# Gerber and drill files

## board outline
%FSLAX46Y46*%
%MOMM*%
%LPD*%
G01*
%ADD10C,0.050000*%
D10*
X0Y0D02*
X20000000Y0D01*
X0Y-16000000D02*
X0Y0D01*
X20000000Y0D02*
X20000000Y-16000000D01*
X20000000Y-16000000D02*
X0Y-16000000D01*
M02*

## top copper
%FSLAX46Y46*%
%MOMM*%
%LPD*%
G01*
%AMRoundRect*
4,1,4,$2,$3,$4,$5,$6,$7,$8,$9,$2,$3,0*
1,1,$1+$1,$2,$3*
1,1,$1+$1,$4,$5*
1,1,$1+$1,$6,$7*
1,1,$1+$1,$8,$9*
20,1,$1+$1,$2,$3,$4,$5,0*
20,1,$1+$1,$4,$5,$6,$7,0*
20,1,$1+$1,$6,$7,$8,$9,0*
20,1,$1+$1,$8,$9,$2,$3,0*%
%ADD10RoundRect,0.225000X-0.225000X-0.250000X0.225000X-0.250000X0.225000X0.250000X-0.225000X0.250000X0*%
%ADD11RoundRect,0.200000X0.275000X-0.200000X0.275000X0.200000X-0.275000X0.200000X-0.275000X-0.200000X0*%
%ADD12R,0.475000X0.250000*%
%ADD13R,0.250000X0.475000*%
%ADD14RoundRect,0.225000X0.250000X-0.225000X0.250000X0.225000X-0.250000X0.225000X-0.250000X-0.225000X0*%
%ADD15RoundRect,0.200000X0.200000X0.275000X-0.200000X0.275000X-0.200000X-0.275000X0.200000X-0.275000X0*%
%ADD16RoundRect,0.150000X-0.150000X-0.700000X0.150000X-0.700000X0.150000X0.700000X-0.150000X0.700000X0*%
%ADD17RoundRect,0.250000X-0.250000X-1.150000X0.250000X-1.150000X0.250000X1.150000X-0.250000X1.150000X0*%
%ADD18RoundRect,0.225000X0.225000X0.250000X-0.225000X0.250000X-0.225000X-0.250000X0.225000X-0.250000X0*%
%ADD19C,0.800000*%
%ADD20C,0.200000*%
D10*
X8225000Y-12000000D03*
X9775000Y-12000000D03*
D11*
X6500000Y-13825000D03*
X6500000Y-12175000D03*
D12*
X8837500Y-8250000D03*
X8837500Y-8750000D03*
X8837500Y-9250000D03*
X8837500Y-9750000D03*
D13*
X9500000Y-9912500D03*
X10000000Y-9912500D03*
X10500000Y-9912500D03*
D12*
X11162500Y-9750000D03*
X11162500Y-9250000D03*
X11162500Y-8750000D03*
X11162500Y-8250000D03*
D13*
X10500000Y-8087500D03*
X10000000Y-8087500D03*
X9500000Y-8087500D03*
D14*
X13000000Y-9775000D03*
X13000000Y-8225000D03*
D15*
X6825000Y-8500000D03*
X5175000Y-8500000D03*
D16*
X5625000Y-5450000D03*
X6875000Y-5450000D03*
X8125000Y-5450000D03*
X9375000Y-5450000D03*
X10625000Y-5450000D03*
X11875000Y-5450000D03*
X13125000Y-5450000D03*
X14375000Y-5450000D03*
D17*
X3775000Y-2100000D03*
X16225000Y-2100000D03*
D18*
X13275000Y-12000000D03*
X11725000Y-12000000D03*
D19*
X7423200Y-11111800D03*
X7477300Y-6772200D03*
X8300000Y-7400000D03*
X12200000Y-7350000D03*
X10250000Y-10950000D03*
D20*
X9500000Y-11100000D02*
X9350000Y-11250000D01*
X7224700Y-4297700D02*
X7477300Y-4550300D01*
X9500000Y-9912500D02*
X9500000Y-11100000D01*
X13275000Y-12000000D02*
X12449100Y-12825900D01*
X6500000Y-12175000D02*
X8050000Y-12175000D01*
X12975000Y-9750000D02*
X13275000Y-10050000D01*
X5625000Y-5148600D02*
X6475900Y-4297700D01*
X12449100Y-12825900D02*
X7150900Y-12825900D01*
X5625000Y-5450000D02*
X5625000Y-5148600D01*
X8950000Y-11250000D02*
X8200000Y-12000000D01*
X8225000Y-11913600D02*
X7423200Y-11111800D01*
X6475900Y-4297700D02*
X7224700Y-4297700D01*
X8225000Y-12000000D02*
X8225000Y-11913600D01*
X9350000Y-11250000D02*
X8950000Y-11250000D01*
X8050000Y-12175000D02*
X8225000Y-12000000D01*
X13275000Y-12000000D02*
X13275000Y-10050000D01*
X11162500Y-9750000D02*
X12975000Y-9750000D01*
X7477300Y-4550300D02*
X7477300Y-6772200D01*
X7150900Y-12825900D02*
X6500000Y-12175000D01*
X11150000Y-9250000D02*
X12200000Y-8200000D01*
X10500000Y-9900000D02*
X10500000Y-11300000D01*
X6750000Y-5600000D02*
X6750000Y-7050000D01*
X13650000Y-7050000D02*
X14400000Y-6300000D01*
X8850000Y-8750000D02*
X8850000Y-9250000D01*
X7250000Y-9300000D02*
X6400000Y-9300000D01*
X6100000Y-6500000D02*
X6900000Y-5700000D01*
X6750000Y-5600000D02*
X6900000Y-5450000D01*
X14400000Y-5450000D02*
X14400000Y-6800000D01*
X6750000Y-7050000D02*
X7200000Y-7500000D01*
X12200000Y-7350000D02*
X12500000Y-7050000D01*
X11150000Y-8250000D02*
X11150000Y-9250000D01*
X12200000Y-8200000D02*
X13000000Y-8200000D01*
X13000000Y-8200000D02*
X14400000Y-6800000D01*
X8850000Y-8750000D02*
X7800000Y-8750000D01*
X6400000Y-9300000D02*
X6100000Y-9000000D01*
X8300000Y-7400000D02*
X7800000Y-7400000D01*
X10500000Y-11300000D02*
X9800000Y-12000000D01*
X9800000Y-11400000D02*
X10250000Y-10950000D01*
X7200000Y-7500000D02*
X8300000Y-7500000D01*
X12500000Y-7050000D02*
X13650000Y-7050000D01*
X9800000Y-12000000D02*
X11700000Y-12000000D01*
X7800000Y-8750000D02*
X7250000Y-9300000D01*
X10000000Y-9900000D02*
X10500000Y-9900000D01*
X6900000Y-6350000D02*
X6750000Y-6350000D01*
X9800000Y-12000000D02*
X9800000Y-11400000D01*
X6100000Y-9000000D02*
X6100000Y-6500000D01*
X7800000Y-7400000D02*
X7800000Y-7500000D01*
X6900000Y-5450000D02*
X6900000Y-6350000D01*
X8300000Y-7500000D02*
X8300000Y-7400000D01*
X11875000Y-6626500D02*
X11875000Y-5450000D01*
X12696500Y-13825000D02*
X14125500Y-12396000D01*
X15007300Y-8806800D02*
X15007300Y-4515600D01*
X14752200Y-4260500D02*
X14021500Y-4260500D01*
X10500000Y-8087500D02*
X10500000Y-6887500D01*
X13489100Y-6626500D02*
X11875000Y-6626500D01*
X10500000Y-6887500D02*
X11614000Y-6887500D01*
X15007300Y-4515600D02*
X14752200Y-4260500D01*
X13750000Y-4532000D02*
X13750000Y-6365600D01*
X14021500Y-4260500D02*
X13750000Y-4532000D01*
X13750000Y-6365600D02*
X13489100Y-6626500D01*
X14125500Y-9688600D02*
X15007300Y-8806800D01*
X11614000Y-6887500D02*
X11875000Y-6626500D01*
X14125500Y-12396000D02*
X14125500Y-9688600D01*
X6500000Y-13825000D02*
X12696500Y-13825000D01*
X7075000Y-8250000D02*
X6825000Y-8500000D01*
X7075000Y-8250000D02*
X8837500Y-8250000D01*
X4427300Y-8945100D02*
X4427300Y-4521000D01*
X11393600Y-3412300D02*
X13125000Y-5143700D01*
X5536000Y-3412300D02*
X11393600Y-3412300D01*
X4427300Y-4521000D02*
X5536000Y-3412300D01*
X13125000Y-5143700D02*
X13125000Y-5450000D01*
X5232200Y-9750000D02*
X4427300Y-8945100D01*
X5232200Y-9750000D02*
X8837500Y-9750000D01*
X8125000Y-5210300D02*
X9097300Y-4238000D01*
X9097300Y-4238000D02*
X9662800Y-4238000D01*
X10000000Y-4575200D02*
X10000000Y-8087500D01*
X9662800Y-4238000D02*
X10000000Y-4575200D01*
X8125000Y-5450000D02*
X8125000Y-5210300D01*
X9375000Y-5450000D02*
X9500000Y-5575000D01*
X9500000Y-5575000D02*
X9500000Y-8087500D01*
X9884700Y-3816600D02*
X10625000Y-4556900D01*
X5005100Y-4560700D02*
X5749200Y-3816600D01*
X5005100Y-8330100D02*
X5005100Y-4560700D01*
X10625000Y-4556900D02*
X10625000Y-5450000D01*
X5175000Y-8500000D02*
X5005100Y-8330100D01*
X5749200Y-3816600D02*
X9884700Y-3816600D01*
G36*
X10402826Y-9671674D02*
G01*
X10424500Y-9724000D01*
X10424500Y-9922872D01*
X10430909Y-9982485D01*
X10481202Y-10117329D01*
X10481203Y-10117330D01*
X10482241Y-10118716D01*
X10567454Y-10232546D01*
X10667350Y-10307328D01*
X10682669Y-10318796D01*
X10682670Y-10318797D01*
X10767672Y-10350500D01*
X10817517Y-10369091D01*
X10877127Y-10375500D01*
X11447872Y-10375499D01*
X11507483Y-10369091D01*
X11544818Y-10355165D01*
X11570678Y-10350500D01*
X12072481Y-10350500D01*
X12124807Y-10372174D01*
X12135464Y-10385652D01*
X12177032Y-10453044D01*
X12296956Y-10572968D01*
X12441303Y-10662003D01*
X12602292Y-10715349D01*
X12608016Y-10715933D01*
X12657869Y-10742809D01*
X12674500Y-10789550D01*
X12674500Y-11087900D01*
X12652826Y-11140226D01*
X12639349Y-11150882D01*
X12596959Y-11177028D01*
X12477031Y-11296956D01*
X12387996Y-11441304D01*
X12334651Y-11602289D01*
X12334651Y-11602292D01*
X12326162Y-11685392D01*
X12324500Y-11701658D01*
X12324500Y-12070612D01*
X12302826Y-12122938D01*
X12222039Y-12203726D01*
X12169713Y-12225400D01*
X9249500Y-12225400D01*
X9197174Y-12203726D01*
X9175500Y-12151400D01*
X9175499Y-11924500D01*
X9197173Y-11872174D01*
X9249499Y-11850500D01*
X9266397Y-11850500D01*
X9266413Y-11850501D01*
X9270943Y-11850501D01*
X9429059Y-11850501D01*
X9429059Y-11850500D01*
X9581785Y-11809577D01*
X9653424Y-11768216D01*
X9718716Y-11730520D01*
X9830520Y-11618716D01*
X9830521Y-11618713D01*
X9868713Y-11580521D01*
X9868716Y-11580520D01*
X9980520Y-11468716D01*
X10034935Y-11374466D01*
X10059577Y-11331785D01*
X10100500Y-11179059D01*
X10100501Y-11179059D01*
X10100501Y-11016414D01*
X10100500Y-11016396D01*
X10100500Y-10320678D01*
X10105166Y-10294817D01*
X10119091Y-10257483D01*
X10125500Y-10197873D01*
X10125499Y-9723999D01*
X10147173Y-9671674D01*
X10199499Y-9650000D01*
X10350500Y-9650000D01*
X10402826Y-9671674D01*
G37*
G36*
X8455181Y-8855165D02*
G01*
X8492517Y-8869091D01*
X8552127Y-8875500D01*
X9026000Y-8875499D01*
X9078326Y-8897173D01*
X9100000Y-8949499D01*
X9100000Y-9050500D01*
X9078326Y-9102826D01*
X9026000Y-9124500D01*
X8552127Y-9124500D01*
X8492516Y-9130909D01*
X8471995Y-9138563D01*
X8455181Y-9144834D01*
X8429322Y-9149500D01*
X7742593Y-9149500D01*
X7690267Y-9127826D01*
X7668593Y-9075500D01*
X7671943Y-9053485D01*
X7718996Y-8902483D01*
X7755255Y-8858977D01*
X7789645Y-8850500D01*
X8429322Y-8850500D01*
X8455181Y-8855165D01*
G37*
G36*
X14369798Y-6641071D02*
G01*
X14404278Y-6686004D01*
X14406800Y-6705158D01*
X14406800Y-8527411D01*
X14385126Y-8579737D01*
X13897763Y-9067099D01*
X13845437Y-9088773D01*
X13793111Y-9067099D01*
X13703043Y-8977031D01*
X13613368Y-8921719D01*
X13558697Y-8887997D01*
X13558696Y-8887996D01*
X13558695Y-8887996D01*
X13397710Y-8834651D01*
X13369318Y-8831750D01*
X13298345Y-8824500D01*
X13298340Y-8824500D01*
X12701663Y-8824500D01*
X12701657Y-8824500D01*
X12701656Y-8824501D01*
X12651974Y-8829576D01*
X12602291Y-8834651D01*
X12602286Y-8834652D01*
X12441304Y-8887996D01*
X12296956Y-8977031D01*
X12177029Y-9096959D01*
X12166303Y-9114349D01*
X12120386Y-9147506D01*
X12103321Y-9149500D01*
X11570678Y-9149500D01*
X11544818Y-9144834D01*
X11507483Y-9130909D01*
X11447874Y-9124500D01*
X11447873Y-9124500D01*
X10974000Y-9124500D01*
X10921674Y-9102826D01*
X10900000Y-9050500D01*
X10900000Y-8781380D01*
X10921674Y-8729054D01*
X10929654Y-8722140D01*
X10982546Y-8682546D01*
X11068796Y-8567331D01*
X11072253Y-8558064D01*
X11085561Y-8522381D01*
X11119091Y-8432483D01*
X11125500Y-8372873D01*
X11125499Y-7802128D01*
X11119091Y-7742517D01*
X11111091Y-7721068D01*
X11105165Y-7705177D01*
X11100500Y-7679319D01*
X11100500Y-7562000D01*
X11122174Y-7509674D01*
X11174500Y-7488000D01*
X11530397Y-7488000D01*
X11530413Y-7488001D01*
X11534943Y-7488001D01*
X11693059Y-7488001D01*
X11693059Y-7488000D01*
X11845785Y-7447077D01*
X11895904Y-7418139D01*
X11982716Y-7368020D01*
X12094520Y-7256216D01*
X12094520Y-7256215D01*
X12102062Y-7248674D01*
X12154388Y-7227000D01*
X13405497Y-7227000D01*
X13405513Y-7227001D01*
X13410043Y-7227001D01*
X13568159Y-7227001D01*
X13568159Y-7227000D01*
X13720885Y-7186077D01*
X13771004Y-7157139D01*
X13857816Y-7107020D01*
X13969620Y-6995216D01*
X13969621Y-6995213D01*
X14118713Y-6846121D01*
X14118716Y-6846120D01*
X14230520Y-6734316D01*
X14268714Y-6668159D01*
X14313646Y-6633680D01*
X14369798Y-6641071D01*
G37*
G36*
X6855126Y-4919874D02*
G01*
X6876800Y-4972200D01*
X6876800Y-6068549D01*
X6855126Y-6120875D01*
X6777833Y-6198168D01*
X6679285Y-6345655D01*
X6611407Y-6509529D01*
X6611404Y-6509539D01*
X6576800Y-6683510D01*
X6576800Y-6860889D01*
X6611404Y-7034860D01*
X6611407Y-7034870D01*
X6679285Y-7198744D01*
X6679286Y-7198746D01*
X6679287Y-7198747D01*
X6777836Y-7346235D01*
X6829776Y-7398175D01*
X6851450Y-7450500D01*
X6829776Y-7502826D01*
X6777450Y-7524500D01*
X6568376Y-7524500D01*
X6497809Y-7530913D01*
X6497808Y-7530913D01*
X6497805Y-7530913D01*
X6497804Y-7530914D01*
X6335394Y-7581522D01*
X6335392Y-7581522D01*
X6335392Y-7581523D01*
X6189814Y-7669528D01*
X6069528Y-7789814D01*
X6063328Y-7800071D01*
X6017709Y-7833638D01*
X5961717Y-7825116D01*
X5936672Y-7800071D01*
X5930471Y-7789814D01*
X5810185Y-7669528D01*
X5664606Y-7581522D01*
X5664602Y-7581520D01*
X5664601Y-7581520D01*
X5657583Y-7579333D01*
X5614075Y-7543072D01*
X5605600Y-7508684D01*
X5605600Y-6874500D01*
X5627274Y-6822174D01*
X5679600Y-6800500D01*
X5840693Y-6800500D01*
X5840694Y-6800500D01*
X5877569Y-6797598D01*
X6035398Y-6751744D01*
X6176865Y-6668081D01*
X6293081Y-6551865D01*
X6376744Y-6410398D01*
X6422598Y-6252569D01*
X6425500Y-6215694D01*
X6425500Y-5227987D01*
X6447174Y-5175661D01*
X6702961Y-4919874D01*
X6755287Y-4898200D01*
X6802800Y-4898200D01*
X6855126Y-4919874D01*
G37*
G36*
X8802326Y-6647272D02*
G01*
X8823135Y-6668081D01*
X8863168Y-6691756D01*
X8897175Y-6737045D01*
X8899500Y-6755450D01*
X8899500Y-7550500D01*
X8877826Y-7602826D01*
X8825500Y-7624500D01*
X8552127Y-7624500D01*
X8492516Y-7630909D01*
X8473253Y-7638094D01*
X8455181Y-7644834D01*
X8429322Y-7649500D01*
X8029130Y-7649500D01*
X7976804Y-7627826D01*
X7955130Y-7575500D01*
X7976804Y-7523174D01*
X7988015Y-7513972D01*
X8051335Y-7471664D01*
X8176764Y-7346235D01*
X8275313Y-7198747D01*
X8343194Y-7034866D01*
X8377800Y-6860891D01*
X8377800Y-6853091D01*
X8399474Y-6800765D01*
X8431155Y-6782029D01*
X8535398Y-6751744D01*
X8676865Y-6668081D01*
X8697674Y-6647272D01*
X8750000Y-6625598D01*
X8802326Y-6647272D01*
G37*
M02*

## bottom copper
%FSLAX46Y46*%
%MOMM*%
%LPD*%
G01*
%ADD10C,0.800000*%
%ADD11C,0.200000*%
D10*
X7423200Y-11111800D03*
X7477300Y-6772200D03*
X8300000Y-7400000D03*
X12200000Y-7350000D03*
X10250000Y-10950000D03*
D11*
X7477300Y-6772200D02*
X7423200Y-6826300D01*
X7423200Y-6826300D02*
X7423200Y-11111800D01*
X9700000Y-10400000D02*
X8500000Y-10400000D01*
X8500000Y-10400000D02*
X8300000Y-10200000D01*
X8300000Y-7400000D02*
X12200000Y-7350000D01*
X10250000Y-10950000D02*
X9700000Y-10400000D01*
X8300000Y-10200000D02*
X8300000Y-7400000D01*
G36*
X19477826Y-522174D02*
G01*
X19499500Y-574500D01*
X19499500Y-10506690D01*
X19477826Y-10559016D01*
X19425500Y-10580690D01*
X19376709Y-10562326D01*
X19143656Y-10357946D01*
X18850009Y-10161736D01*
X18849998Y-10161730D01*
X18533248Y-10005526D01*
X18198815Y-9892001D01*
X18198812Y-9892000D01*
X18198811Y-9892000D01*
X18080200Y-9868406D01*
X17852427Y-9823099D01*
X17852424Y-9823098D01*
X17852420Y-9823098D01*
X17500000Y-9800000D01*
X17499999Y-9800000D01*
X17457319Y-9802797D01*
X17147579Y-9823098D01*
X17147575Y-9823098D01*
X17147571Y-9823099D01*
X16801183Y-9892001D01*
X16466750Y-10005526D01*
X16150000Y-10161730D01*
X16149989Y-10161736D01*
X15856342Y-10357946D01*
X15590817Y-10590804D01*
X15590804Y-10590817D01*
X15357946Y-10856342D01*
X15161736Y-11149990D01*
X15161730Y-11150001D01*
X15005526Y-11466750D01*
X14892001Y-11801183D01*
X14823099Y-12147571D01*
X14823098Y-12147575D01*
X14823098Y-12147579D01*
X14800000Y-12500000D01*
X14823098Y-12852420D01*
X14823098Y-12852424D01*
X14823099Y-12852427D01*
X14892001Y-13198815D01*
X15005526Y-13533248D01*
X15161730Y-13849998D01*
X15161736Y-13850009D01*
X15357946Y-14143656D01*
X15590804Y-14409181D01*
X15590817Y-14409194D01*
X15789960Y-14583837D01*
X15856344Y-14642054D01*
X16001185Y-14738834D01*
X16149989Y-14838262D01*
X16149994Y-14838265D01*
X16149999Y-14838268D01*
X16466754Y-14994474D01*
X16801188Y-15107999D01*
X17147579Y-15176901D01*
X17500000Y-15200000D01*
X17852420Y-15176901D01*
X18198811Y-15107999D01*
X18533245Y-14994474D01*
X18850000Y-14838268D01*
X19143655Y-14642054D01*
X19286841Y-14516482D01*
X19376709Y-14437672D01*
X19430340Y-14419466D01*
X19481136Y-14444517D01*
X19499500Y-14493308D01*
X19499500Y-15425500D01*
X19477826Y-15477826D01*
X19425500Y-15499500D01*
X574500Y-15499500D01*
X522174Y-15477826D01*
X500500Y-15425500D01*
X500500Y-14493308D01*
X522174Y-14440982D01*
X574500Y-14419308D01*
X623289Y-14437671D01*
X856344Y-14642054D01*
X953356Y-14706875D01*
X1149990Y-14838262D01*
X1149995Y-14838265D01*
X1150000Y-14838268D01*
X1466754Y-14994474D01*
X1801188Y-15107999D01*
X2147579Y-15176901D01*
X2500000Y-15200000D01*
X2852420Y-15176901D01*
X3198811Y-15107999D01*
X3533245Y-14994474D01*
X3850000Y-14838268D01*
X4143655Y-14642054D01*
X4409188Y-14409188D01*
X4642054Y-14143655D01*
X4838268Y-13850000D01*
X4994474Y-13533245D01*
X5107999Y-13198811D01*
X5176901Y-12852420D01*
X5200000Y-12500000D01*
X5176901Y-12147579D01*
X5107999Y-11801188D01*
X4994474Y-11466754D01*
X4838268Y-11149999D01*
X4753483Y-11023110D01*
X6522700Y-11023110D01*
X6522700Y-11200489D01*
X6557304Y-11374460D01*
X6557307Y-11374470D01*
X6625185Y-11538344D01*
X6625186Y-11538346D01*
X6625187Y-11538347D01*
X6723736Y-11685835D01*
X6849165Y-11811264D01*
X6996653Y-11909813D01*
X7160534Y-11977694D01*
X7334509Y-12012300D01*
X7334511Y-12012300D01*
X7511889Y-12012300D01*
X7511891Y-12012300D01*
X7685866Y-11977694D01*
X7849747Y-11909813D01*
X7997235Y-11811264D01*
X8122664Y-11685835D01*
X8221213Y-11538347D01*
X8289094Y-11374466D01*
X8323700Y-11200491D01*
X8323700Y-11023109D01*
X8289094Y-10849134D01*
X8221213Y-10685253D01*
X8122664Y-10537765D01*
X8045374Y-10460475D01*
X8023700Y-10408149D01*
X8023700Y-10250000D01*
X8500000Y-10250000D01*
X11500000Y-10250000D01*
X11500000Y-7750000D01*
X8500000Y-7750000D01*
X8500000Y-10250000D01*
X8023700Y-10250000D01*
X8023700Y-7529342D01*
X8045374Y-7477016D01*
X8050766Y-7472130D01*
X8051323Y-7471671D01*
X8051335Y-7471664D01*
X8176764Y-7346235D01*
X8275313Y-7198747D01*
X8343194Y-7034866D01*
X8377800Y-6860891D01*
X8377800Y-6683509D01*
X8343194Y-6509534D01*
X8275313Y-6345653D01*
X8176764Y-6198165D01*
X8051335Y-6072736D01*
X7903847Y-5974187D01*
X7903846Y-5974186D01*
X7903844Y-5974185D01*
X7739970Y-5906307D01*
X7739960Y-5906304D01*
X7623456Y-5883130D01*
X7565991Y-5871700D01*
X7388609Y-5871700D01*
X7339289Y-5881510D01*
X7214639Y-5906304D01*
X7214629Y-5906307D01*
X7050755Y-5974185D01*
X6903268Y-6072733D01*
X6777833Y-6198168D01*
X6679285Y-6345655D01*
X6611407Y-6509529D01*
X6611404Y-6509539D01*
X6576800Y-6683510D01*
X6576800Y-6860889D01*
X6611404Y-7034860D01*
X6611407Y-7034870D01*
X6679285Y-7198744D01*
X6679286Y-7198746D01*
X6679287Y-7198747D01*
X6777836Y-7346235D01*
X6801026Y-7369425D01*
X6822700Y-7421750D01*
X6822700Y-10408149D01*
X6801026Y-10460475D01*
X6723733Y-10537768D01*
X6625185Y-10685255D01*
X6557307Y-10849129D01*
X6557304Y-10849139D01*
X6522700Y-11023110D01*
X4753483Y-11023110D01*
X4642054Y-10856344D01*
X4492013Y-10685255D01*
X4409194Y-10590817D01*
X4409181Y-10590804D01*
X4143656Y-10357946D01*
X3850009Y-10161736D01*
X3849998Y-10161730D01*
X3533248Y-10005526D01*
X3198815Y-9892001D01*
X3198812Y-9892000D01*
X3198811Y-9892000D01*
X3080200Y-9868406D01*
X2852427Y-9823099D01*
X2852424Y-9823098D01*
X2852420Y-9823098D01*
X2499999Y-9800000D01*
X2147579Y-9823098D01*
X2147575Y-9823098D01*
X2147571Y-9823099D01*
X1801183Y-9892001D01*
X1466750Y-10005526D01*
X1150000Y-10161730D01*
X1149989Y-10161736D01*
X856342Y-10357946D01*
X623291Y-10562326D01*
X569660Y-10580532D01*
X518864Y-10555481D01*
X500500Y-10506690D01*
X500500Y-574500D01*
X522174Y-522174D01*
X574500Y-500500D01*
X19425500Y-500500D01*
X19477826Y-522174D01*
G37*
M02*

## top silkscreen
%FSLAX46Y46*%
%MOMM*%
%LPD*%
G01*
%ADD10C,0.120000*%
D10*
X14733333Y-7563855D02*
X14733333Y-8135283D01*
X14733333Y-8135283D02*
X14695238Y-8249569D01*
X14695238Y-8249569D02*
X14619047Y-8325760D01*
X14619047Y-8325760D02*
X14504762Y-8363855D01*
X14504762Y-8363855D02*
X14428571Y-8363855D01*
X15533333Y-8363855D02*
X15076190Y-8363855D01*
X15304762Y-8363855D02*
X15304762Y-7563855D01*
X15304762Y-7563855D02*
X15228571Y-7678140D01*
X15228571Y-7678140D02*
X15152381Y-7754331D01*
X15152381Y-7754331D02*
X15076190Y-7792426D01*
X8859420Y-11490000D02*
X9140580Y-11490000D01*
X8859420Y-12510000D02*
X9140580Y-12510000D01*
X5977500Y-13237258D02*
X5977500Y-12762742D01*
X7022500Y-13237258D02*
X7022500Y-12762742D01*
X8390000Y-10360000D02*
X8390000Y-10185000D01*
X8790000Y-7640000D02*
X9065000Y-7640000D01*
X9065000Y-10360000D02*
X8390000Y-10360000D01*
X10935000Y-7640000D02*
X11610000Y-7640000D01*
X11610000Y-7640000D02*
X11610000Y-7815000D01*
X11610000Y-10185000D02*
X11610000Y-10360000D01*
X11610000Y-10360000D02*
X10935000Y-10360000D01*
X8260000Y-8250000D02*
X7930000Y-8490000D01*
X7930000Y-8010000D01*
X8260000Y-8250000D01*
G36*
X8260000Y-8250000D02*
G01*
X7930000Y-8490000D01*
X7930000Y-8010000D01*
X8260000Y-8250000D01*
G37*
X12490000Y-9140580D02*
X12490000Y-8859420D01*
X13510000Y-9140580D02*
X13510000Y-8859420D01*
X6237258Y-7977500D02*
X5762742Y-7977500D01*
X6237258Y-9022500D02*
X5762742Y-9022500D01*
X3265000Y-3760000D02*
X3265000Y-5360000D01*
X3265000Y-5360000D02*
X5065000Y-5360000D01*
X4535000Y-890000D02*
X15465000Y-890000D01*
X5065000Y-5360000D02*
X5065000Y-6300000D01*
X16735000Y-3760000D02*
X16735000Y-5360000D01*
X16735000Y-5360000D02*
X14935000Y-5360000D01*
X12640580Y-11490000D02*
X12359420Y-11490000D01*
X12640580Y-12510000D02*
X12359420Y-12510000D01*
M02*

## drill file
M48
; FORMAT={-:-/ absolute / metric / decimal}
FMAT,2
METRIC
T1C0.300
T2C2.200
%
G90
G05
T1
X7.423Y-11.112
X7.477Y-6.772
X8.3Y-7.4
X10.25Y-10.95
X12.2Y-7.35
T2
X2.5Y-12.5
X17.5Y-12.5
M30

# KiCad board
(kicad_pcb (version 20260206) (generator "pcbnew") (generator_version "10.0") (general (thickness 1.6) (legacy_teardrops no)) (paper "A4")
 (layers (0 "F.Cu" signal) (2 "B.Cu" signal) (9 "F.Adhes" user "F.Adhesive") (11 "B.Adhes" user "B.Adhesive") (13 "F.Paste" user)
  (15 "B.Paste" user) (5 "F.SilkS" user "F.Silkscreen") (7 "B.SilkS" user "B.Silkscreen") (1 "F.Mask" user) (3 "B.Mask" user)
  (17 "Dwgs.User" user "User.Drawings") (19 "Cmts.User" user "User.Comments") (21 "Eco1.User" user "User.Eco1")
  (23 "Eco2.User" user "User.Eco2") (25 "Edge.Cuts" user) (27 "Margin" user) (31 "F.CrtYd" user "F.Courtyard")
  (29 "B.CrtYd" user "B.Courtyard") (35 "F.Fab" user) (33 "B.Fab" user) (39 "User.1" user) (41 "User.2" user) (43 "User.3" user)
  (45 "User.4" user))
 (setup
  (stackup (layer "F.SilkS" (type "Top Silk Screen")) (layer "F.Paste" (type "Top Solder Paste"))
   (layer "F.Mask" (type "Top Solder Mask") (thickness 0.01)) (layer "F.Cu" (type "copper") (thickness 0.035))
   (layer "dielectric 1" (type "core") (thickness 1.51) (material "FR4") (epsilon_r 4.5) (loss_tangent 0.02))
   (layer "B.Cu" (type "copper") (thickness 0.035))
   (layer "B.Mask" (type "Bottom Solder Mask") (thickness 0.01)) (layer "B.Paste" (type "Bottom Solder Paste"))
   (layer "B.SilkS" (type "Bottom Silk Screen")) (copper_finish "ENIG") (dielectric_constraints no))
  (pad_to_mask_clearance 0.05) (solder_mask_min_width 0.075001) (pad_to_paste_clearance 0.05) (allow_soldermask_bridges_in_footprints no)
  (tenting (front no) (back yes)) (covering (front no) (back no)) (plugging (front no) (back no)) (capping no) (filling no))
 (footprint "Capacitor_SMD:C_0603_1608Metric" (layer "F.Cu") (at 9 12)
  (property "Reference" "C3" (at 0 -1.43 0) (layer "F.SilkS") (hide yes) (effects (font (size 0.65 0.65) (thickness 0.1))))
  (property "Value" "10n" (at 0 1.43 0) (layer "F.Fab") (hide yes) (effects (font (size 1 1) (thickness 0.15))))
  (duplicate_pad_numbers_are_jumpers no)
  (fp_line (start -0.14058 -0.51) (end 0.14058 -0.51) (stroke (width 0.12) (type solid)) (layer "F.SilkS"))
  (fp_line (start -0.14058 0.51) (end 0.14058 0.51) (stroke (width 0.12) (type solid)) (layer "F.SilkS"))
  (pad "1" smd roundrect (at -0.775 0) (size 0.9 0.95) (layers "F.Cu" "F.Mask" "F.Paste") (roundrect_rratio 0.25) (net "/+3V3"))
  (pad "2" smd roundrect (at 0.775 0) (size 0.9 0.95) (layers "F.Cu" "F.Mask" "F.Paste") (roundrect_rratio 0.25) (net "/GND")
   (zone_connect 2)))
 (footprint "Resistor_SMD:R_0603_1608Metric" (layer "F.Cu") (at 6.5 13 90)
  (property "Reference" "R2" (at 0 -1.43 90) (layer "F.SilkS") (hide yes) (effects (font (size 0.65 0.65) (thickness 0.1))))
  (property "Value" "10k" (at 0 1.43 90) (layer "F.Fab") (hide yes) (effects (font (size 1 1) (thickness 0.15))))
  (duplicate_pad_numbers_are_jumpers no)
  (fp_line (start -0.237258 -0.5225) (end 0.237258 -0.5225) (stroke (width 0.12) (type solid)) (layer "F.SilkS"))
  (fp_line (start -0.237258 0.5225) (end 0.237258 0.5225) (stroke (width 0.12) (type solid)) (layer "F.SilkS"))
  (pad "1" smd roundrect (at -0.825 0 90) (size 0.8 0.95) (layers "F.Cu" "F.Mask" "F.Paste") (roundrect_rratio 0.25) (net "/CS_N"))
  (pad "2" smd roundrect (at 0.825 0 90) (size 0.8 0.95) (layers "F.Cu" "F.Mask" "F.Paste") (roundrect_rratio 0.25) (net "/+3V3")))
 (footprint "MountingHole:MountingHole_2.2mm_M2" (layer "F.Cu") (at 2.5 12.5)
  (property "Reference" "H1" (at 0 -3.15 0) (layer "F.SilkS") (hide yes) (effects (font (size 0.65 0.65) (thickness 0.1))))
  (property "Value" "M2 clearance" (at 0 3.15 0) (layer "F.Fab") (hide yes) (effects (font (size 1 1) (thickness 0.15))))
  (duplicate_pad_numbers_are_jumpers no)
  (pad "" np_thru_hole circle (at 0 0) (size 2.2 2.2) (drill 2.2) (layers "*.Cu" "*.Mask")))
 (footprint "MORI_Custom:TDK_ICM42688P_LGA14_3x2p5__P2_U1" (layer "F.Cu") (at 10 9)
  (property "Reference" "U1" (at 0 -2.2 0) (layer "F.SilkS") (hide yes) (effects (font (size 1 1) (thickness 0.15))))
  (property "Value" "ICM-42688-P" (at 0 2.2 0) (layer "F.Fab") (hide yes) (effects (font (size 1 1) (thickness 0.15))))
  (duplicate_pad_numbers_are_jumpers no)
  (fp_line (start -1.61 1.36) (end -1.61 1.185) (stroke (width 0.12) (type solid)) (layer "F.SilkS"))
  (fp_line (start -1.21 -1.36) (end -0.935 -1.36) (stroke (width 0.12) (type default)) (layer "F.SilkS"))
  (fp_line (start -0.935 1.36) (end -1.61 1.36) (stroke (width 0.12) (type solid)) (layer "F.SilkS"))
  (fp_line (start 0.935 -1.36) (end 1.61 -1.36) (stroke (width 0.12) (type solid)) (layer "F.SilkS"))
  (fp_line (start 1.61 -1.36) (end 1.61 -1.185) (stroke (width 0.12) (type solid)) (layer "F.SilkS"))
  (fp_line (start 1.61 1.185) (end 1.61 1.36) (stroke (width 0.12) (type solid)) (layer "F.SilkS"))
  (fp_line (start 1.61 1.36) (end 0.935 1.36) (stroke (width 0.12) (type solid)) (layer "F.SilkS"))
  (fp_poly (pts (xy -1.74 -0.75) (xy -2.07 -0.51) (xy -2.07 -0.99)) (stroke (width 0.12) (type solid)) (fill yes) (layer "F.SilkS"))
  (pad "1" smd rect (at -1.1625 -0.75) (size 0.475 0.25) (layers "F.Cu" "F.Mask" "F.Paste") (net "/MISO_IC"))
  (pad "2" smd rect (at -1.1625 -0.25) (size 0.475 0.25) (layers "F.Cu" "F.Mask" "F.Paste") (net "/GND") (zone_connect 2))
  (pad "3" smd rect (at -1.1625 0.25) (size 0.475 0.25) (layers "F.Cu" "F.Mask" "F.Paste") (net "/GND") (zone_connect 2))
  (pad "4" smd rect (at -1.1625 0.75) (size 0.475 0.25) (layers "F.Cu" "F.Mask" "F.Paste") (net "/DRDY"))
  (pad "5" smd rect (at -0.5 0.9125) (size 0.25 0.475) (layers "F.Cu" "F.Mask" "F.Paste") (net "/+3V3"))
  (pad "6" smd rect (at 0 0.9125) (size 0.25 0.475) (layers "F.Cu" "F.Mask" "F.Paste") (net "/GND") (zone_connect 2))
  (pad "7" smd rect (at 0.5 0.9125) (size 0.25 0.475) (layers "F.Cu" "F.Mask" "F.Paste") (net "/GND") (zone_connect 2))
  (pad "8" smd rect (at 1.1625 0.75) (size 0.475 0.25) (layers "F.Cu" "F.Mask" "F.Paste") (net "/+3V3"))
  (pad "9" smd rect (at 1.1625 0.25) (size 0.475 0.25) (layers "F.Cu" "F.Mask" "F.Paste") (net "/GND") (zone_connect 2))
  (pad "10" smd rect (at 1.1625 -0.25) (size 0.475 0.25) (layers "F.Cu" "F.Mask" "F.Paste") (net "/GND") (zone_connect 2))
  (pad "11" smd rect (at 1.1625 -0.75) (size 0.475 0.25) (layers "F.Cu" "F.Mask" "F.Paste") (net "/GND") (zone_connect 2))
  (pad "12" smd rect (at 0.5 -0.9125) (size 0.25 0.475) (layers "F.Cu" "F.Mask" "F.Paste") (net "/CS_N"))
  (pad "13" smd rect (at 0 -0.9125) (size 0.25 0.475) (layers "F.Cu" "F.Mask" "F.Paste") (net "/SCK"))
  (pad "14" smd rect (at -0.5 -0.9125) (size 0.25 0.475) (layers "F.Cu" "F.Mask" "F.Paste") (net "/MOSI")))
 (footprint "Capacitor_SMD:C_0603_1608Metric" (layer "F.Cu") (at 13 9 90)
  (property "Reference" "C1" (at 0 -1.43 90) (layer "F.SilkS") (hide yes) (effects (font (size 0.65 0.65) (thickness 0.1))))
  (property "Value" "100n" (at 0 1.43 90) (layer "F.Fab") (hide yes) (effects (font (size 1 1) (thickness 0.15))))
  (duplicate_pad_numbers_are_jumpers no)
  (fp_line (start -0.14058 -0.51) (end 0.14058 -0.51) (stroke (width 0.12) (type solid)) (layer "F.SilkS"))
  (fp_line (start -0.14058 0.51) (end 0.14058 0.51) (stroke (width 0.12) (type solid)) (layer "F.SilkS"))
  (pad "1" smd roundrect (at -0.775 0 90) (size 0.9 0.95) (layers "F.Cu" "F.Mask" "F.Paste") (roundrect_rratio 0.25) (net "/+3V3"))
  (pad "2" smd roundrect (at 0.775 0 90) (size 0.9 0.95) (layers "F.Cu" "F.Mask" "F.Paste") (roundrect_rratio 0.25) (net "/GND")
   (zone_connect 2)))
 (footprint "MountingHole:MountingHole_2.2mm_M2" (layer "F.Cu") (at 17.5 12.5)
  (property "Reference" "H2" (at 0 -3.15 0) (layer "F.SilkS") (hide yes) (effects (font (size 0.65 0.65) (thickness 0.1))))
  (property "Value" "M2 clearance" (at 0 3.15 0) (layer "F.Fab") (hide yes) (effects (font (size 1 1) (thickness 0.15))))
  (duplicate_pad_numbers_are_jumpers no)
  (pad "" np_thru_hole circle (at 0 0) (size 2.2 2.2) (drill 2.2) (layers "*.Cu" "*.Mask")))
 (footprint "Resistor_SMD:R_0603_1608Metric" (layer "F.Cu") (at 6 8.5 180)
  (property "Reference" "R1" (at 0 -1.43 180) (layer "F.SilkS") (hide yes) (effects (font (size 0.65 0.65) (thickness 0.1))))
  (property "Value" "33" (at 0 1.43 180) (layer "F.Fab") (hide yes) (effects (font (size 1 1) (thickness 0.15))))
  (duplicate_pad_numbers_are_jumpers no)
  (fp_line (start -0.237258 0.5225) (end 0.237258 0.5225) (stroke (width 0.12) (type solid)) (layer "F.SilkS"))
  (fp_line (start -0.237258 -0.5225) (end 0.237258 -0.5225) (stroke (width 0.12) (type solid)) (layer "F.SilkS"))
  (pad "1" smd roundrect (at -0.825 0 180) (size 0.8 0.95) (layers "F.Cu" "F.Mask" "F.Paste") (roundrect_rratio 0.25) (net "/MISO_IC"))
  (pad "2" smd roundrect (at 0.825 0 180) (size 0.8 0.95) (layers "F.Cu" "F.Mask" "F.Paste") (roundrect_rratio 0.25) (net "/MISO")))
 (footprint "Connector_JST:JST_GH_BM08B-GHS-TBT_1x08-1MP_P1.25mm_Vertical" (layer "F.Cu") (at 10 3.5)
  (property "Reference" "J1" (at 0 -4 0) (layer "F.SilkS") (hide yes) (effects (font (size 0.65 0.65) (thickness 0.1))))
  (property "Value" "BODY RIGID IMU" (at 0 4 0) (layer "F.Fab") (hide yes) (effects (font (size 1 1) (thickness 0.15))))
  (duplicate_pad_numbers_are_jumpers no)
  (fp_line (start -6.735 0.26) (end -6.735 1.86) (stroke (width 0.12) (type solid)) (layer "F.SilkS"))
  (fp_line (start -6.735 1.86) (end -4.935 1.86) (stroke (width 0.12) (type solid)) (layer "F.SilkS"))
  (fp_line (start -5.465 -2.61) (end 5.465 -2.61) (stroke (width 0.12) (type solid)) (layer "F.SilkS"))
  (fp_line (start -4.935 1.86) (end -4.935 2.8) (stroke (width 0.12) (type solid)) (layer "F.SilkS"))
  (fp_line (start 6.735 0.26) (end 6.735 1.86) (stroke (width 0.12) (type solid)) (layer "F.SilkS"))
  (fp_line (start 6.735 1.86) (end 4.935 1.86) (stroke (width 0.12) (type solid)) (layer "F.SilkS"))
  (pad "1" smd roundrect (at -4.375 1.95) (size 0.6 1.7) (layers "F.Cu" "F.Mask" "F.Paste") (roundrect_rratio 0.25) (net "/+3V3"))
  (pad "2" smd roundrect (at -3.125 1.95) (size 0.6 1.7) (layers "F.Cu" "F.Mask" "F.Paste") (roundrect_rratio 0.25) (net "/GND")
   (zone_connect 2))
  (pad "3" smd roundrect (at -1.875 1.95) (size 0.6 1.7) (layers "F.Cu" "F.Mask" "F.Paste") (roundrect_rratio 0.25) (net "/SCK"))
  (pad "4" smd roundrect (at -0.625 1.95) (size 0.6 1.7) (layers "F.Cu" "F.Mask" "F.Paste") (roundrect_rratio 0.25) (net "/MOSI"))
  (pad "5" smd roundrect (at 0.625 1.95) (size 0.6 1.7) (layers "F.Cu" "F.Mask" "F.Paste") (roundrect_rratio 0.25) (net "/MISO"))
  (pad "6" smd roundrect (at 1.875 1.95) (size 0.6 1.7) (layers "F.Cu" "F.Mask" "F.Paste") (roundrect_rratio 0.25) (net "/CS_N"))
  (pad "7" smd roundrect (at 3.125 1.95) (size 0.6 1.7) (layers "F.Cu" "F.Mask" "F.Paste") (roundrect_rratio 0.25) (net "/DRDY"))
  (pad "8" smd roundrect (at 4.375 1.95) (size 0.6 1.7) (layers "F.Cu" "F.Mask" "F.Paste") (roundrect_rratio 0.25) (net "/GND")
   (zone_connect 2))
  (pad "MP" smd roundrect (at -6.225 -1.4) (size 1 2.8) (layers "F.Cu" "F.Mask" "F.Paste") (roundrect_rratio 0.25))
  (pad "MP" smd roundrect (at 6.225 -1.4) (size 1 2.8) (layers "F.Cu" "F.Mask" "F.Paste") (roundrect_rratio 0.25)))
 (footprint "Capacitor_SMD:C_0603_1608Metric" (layer "F.Cu") (at 12.5 12 180)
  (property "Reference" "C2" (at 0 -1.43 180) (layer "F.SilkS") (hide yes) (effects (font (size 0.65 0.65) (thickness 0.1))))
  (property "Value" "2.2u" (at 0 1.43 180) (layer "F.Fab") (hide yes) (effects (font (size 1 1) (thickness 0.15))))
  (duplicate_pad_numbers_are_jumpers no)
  (fp_line (start -0.14058 0.51) (end 0.14058 0.51) (stroke (width 0.12) (type solid)) (layer "F.SilkS"))
  (fp_line (start -0.14058 -0.51) (end 0.14058 -0.51) (stroke (width 0.12) (type solid)) (layer "F.SilkS"))
  (pad "1" smd roundrect (at -0.775 0 180) (size 0.9 0.95) (layers "F.Cu" "F.Mask" "F.Paste") (roundrect_rratio 0.25) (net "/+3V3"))
  (pad "2" smd roundrect (at 0.775 0 180) (size 0.9 0.95) (layers "F.Cu" "F.Mask" "F.Paste") (roundrect_rratio 0.25) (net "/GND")
   (zone_connect 2)))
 (gr_line (start 0 0) (end 20 0) (stroke (width 0.05) (type default)) (layer "Edge.Cuts"))
 (gr_line (start 0 16) (end 0 0) (stroke (width 0.05) (type default)) (layer "Edge.Cuts"))
 (gr_line (start 20 0) (end 20 16) (stroke (width 0.05) (type default)) (layer "Edge.Cuts"))
 (gr_line (start 20 16) (end 0 16) (stroke (width 0.05) (type default)) (layer "Edge.Cuts"))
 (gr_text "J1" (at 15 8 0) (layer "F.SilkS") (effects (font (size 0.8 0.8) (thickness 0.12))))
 (segment (start 9.5 11.1) (end 9.35 11.25) (width 0.2) (layer "F.Cu") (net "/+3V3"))
 (segment (start 7.2247 4.2977) (end 7.4773 4.5503) (width 0.2) (layer "F.Cu") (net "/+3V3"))
 (segment (start 9.5 9.9125) (end 9.5 11.1) (width 0.2) (layer "F.Cu") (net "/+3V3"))
 (segment (start 13.275 12) (end 12.4491 12.8259) (width 0.2) (layer "F.Cu") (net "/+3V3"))
 (segment (start 6.5 12.175) (end 8.05 12.175) (width 0.2) (layer "F.Cu") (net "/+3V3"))
 (segment (start 12.975 9.75) (end 13.275 10.05) (width 0.2) (layer "F.Cu") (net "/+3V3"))
 (segment (start 5.625 5.1486) (end 6.4759 4.2977) (width 0.2) (layer "F.Cu") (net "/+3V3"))
 (segment (start 12.4491 12.8259) (end 7.1509 12.8259) (width 0.2) (layer "F.Cu") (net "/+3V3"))
 (segment (start 5.625 5.45) (end 5.625 5.1486) (width 0.2) (layer "F.Cu") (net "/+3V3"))
 (segment (start 8.95 11.25) (end 8.2 12) (width 0.2) (layer "F.Cu") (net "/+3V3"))
 (segment (start 8.225 11.9136) (end 7.4232 11.1118) (width 0.2) (layer "F.Cu") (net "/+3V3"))
 (segment (start 6.4759 4.2977) (end 7.2247 4.2977) (width 0.2) (layer "F.Cu") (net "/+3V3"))
 (segment (start 8.225 12) (end 8.225 11.9136) (width 0.2) (layer "F.Cu") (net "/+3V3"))
 (segment (start 9.35 11.25) (end 8.95 11.25) (width 0.2) (layer "F.Cu") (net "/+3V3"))
 (segment (start 8.05 12.175) (end 8.225 12) (width 0.2) (layer "F.Cu") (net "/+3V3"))
 (segment (start 13.275 12) (end 13.275 10.05) (width 0.2) (layer "F.Cu") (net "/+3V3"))
 (segment (start 11.1625 9.75) (end 12.975 9.75) (width 0.2) (layer "F.Cu") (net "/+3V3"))
 (segment (start 7.4773 4.5503) (end 7.4773 6.7722) (width 0.2) (layer "F.Cu") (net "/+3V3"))
 (segment (start 7.1509 12.8259) (end 6.5 12.175) (width 0.2) (layer "F.Cu") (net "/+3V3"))
 (via (at 7.4232 11.1118) (size 0.8) (drill 0.3) (layers "F.Cu" "B.Cu") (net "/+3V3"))
 (via (at 7.4773 6.7722) (size 0.8) (drill 0.3) (layers "F.Cu" "B.Cu") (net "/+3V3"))
 (segment (start 7.4773 6.7722) (end 7.4232 6.8263) (width 0.2) (layer "B.Cu") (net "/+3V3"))
 (segment (start 7.4232 6.8263) (end 7.4232 11.1118) (width 0.2) (layer "B.Cu") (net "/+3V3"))
 (segment (start 11.15 9.25) (end 12.2 8.2) (width 0.2) (layer "F.Cu") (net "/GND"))
 (segment (start 10.5 9.9) (end 10.5 11.3) (width 0.2) (layer "F.Cu") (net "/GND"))
 (segment (start 6.75 5.6) (end 6.75 7.05) (width 0.2) (layer "F.Cu") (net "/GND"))
 (segment (start 13.65 7.05) (end 14.4 6.3) (width 0.2) (layer "F.Cu") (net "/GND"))
 (segment (start 8.85 8.75) (end 8.85 9.25) (width 0.2) (layer "F.Cu") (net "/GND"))
 (segment (start 7.25 9.3) (end 6.4 9.3) (width 0.2) (layer "F.Cu") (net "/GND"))
 (segment (start 6.1 6.5) (end 6.9 5.7) (width 0.2) (layer "F.Cu") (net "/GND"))
 (segment (start 6.75 5.6) (end 6.9 5.45) (width 0.2) (layer "F.Cu") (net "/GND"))
 (segment (start 14.4 5.45) (end 14.4 6.8) (width 0.2) (layer "F.Cu") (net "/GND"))
 (segment (start 6.75 7.05) (end 7.2 7.5) (width 0.2) (layer "F.Cu") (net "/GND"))
 (segment (start 12.2 7.35) (end 12.5 7.05) (width 0.2) (layer "F.Cu") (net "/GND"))
 (segment (start 11.15 8.25) (end 11.15 9.25) (width 0.2) (layer "F.Cu") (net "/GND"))
 (segment (start 12.2 8.2) (end 13 8.2) (width 0.2) (layer "F.Cu") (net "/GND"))
 (segment (start 13 8.2) (end 14.4 6.8) (width 0.2) (layer "F.Cu") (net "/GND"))
 (segment (start 8.85 8.75) (end 7.8 8.75) (width 0.2) (layer "F.Cu") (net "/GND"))
 (segment (start 6.4 9.3) (end 6.1 9) (width 0.2) (layer "F.Cu") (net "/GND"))
 (segment (start 8.3 7.4) (end 7.8 7.4) (width 0.2) (layer "F.Cu") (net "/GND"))
 (segment (start 10.5 11.3) (end 9.8 12) (width 0.2) (layer "F.Cu") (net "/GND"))
 (segment (start 9.8 11.4) (end 10.25 10.95) (width 0.2) (layer "F.Cu") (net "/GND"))
 (segment (start 7.2 7.5) (end 8.3 7.5) (width 0.2) (layer "F.Cu") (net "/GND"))
 (segment (start 12.5 7.05) (end 13.65 7.05) (width 0.2) (layer "F.Cu") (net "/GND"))
 (segment (start 9.8 12) (end 11.7 12) (width 0.2) (layer "F.Cu") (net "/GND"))
 (segment (start 7.8 8.75) (end 7.25 9.3) (width 0.2) (layer "F.Cu") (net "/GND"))
 (segment (start 10 9.9) (end 10.5 9.9) (width 0.2) (layer "F.Cu") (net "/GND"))
 (segment (start 6.9 6.35) (end 6.75 6.35) (width 0.2) (layer "F.Cu") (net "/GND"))
 (segment (start 9.8 12) (end 9.8 11.4) (width 0.2) (layer "F.Cu") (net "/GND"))
 (segment (start 6.1 9) (end 6.1 6.5) (width 0.2) (layer "F.Cu") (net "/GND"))
 (segment (start 7.8 7.4) (end 7.8 7.5) (width 0.2) (layer "F.Cu") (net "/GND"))
 (segment (start 6.9 5.45) (end 6.9 6.35) (width 0.2) (layer "F.Cu") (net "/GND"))
 (segment (start 8.3 7.5) (end 8.3 7.4) (width 0.2) (layer "F.Cu") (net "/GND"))
 (via (at 8.3 7.4) (size 0.8) (drill 0.3) (layers "F.Cu" "B.Cu") (tenting (front no) (back none)) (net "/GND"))
 (via (at 12.2 7.35) (size 0.8) (drill 0.3) (layers "F.Cu" "B.Cu") (tenting (front no) (back none)) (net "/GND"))
 (via (at 10.25 10.95) (size 0.8) (drill 0.3) (layers "F.Cu" "B.Cu") (tenting (front no) (back none)) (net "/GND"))
 (segment (start 9.7 10.4) (end 8.5 10.4) (width 0.2) (layer "B.Cu") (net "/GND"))
 (segment (start 8.5 10.4) (end 8.3 10.2) (width 0.2) (layer "B.Cu") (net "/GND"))
 (segment (start 8.3 7.4) (end 12.2 7.35) (width 0.2) (layer "B.Cu") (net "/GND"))
 (segment (start 10.25 10.95) (end 9.7 10.4) (width 0.2) (layer "B.Cu") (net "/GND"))
 (segment (start 8.3 10.2) (end 8.3 7.4) (width 0.2) (layer "B.Cu") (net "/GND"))
 (segment (start 11.875 6.6265) (end 11.875 5.45) (width 0.2) (layer "F.Cu") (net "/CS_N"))
 (segment (start 12.6965 13.825) (end 14.1255 12.396) (width 0.2) (layer "F.Cu") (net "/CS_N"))
 (segment (start 15.0073 8.8068) (end 15.0073 4.5156) (width 0.2) (layer "F.Cu") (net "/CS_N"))
 (segment (start 14.7522 4.2605) (end 14.0215 4.2605) (width 0.2) (layer "F.Cu") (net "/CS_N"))
 (segment (start 10.5 8.0875) (end 10.5 6.8875) (width 0.2) (layer "F.Cu") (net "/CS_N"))
 (segment (start 13.4891 6.6265) (end 11.875 6.6265) (width 0.2) (layer "F.Cu") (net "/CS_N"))
 (segment (start 10.5 6.8875) (end 11.614 6.8875) (width 0.2) (layer "F.Cu") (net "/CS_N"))
 (segment (start 15.0073 4.5156) (end 14.7522 4.2605) (width 0.2) (layer "F.Cu") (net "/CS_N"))
 (segment (start 13.75 4.532) (end 13.75 6.3656) (width 0.2) (layer "F.Cu") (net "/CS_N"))
 (segment (start 14.0215 4.2605) (end 13.75 4.532) (width 0.2) (layer "F.Cu") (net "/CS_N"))
 (segment (start 13.75 6.3656) (end 13.4891 6.6265) (width 0.2) (layer "F.Cu") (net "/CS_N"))
 (segment (start 14.1255 9.6886) (end 15.0073 8.8068) (width 0.2) (layer "F.Cu") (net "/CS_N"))
 (segment (start 11.614 6.8875) (end 11.875 6.6265) (width 0.2) (layer "F.Cu") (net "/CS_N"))
 (segment (start 14.1255 12.396) (end 14.1255 9.6886) (width 0.2) (layer "F.Cu") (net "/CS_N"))
 (segment (start 6.5 13.825) (end 12.6965 13.825) (width 0.2) (layer "F.Cu") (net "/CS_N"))
 (segment (start 7.075 8.25) (end 6.825 8.5) (width 0.2) (layer "F.Cu") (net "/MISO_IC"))
 (segment (start 7.075 8.25) (end 8.8375 8.25) (width 0.2) (layer "F.Cu") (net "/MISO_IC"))
 (segment (start 4.4273 8.9451) (end 4.4273 4.521) (width 0.2) (layer "F.Cu") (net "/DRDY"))
 (segment (start 11.3936 3.4123) (end 13.125 5.1437) (width 0.2) (layer "F.Cu") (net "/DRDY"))
 (segment (start 5.536 3.4123) (end 11.3936 3.4123) (width 0.2) (layer "F.Cu") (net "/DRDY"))
 (segment (start 4.4273 4.521) (end 5.536 3.4123) (width 0.2) (layer "F.Cu") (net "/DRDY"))
 (segment (start 13.125 5.1437) (end 13.125 5.45) (width 0.2) (layer "F.Cu") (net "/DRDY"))
 (segment (start 5.2322 9.75) (end 4.4273 8.9451) (width 0.2) (layer "F.Cu") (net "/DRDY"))
 (segment (start 5.2322 9.75) (end 8.8375 9.75) (width 0.2) (layer "F.Cu") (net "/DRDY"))
 (segment (start 8.125 5.2103) (end 9.0973 4.238) (width 0.2) (layer "F.Cu") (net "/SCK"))
 (segment (start 9.0973 4.238) (end 9.6628 4.238) (width 0.2) (layer "F.Cu") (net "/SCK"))
 (segment (start 10 4.5752) (end 10 8.0875) (width 0.2) (layer "F.Cu") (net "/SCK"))
 (segment (start 9.6628 4.238) (end 10 4.5752) (width 0.2) (layer "F.Cu") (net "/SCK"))
 (segment (start 8.125 5.45) (end 8.125 5.2103) (width 0.2) (layer "F.Cu") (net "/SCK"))
 (segment (start 9.375 5.45) (end 9.5 5.575) (width 0.2) (layer "F.Cu") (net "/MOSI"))
 (segment (start 9.5 5.575) (end 9.5 8.0875) (width 0.2) (layer "F.Cu") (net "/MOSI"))
 (segment (start 9.8847 3.8166) (end 10.625 4.5569) (width 0.2) (layer "F.Cu") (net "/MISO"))
 (segment (start 5.0051 4.5607) (end 5.7492 3.8166) (width 0.2) (layer "F.Cu") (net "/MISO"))
 (segment (start 5.0051 8.3301) (end 5.0051 4.5607) (width 0.2) (layer "F.Cu") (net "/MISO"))
 (segment (start 10.625 4.5569) (end 10.625 5.45) (width 0.2) (layer "F.Cu") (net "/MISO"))
 (segment (start 5.175 8.5) (end 5.0051 8.3301) (width 0.2) (layer "F.Cu") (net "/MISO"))
 (segment (start 5.7492 3.8166) (end 9.8847 3.8166) (width 0.2) (layer "F.Cu") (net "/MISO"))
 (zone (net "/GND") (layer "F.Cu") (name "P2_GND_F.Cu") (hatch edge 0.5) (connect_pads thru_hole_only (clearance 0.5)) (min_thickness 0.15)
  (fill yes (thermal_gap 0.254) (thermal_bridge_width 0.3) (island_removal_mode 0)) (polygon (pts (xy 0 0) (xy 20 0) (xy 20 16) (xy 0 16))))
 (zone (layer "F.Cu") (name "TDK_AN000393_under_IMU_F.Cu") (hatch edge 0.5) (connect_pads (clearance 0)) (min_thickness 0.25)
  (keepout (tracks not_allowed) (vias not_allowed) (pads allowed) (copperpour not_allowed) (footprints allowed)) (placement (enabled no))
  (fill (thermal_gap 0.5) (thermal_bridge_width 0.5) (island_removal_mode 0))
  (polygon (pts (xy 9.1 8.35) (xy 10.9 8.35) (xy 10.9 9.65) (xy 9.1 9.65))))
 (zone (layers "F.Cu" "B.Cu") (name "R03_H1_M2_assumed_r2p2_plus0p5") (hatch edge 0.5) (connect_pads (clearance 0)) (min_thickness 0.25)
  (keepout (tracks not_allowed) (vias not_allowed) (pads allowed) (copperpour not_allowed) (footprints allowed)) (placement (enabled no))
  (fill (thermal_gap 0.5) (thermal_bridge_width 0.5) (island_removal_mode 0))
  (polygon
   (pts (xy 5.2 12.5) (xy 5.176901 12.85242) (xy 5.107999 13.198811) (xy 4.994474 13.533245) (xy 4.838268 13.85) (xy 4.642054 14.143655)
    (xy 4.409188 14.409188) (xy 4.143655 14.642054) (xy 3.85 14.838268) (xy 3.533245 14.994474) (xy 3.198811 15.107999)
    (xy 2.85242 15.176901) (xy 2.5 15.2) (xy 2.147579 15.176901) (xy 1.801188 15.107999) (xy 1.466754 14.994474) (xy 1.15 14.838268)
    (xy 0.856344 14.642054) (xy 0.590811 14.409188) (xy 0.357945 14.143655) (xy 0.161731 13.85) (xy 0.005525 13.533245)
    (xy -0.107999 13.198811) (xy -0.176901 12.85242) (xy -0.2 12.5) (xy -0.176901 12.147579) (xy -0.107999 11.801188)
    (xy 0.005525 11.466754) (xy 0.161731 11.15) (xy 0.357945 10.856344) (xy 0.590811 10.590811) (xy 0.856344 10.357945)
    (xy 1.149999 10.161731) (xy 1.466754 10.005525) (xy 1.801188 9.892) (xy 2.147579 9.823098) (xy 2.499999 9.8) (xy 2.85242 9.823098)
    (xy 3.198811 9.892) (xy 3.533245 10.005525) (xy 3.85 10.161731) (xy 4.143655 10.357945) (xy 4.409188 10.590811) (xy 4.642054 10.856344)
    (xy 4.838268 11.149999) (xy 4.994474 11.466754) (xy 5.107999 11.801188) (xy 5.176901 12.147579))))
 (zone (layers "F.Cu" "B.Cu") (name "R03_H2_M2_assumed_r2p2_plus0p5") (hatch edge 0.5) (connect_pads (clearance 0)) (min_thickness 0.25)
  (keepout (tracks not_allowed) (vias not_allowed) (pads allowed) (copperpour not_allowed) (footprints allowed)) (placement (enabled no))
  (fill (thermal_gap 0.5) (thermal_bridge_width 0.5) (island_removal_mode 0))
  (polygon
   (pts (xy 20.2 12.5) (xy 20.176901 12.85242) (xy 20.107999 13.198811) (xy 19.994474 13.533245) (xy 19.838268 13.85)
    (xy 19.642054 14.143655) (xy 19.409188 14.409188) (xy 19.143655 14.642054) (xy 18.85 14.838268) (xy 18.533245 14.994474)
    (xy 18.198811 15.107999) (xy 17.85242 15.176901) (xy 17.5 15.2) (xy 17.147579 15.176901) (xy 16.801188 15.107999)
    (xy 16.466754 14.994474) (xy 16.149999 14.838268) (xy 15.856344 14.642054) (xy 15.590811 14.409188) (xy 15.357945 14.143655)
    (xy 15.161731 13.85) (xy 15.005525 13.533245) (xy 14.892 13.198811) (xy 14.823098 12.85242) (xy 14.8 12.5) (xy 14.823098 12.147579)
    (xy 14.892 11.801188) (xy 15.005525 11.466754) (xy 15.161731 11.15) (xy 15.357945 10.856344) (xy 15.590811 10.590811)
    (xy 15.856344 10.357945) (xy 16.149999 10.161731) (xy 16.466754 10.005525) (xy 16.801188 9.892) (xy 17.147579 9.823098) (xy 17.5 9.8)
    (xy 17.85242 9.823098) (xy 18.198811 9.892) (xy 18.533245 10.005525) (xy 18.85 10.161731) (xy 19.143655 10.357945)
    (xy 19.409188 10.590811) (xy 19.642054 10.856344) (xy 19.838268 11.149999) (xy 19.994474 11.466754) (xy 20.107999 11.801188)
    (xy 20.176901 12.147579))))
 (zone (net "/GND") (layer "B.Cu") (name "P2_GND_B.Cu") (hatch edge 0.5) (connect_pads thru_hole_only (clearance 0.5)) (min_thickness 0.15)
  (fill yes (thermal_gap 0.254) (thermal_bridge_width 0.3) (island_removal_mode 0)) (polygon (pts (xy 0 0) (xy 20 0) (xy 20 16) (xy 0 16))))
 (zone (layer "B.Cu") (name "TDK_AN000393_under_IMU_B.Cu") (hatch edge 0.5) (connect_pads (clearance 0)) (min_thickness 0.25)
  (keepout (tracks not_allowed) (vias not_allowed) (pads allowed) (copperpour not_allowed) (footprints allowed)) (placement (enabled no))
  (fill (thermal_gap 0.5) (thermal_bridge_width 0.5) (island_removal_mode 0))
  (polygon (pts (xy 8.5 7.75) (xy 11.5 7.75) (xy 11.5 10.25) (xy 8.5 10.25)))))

